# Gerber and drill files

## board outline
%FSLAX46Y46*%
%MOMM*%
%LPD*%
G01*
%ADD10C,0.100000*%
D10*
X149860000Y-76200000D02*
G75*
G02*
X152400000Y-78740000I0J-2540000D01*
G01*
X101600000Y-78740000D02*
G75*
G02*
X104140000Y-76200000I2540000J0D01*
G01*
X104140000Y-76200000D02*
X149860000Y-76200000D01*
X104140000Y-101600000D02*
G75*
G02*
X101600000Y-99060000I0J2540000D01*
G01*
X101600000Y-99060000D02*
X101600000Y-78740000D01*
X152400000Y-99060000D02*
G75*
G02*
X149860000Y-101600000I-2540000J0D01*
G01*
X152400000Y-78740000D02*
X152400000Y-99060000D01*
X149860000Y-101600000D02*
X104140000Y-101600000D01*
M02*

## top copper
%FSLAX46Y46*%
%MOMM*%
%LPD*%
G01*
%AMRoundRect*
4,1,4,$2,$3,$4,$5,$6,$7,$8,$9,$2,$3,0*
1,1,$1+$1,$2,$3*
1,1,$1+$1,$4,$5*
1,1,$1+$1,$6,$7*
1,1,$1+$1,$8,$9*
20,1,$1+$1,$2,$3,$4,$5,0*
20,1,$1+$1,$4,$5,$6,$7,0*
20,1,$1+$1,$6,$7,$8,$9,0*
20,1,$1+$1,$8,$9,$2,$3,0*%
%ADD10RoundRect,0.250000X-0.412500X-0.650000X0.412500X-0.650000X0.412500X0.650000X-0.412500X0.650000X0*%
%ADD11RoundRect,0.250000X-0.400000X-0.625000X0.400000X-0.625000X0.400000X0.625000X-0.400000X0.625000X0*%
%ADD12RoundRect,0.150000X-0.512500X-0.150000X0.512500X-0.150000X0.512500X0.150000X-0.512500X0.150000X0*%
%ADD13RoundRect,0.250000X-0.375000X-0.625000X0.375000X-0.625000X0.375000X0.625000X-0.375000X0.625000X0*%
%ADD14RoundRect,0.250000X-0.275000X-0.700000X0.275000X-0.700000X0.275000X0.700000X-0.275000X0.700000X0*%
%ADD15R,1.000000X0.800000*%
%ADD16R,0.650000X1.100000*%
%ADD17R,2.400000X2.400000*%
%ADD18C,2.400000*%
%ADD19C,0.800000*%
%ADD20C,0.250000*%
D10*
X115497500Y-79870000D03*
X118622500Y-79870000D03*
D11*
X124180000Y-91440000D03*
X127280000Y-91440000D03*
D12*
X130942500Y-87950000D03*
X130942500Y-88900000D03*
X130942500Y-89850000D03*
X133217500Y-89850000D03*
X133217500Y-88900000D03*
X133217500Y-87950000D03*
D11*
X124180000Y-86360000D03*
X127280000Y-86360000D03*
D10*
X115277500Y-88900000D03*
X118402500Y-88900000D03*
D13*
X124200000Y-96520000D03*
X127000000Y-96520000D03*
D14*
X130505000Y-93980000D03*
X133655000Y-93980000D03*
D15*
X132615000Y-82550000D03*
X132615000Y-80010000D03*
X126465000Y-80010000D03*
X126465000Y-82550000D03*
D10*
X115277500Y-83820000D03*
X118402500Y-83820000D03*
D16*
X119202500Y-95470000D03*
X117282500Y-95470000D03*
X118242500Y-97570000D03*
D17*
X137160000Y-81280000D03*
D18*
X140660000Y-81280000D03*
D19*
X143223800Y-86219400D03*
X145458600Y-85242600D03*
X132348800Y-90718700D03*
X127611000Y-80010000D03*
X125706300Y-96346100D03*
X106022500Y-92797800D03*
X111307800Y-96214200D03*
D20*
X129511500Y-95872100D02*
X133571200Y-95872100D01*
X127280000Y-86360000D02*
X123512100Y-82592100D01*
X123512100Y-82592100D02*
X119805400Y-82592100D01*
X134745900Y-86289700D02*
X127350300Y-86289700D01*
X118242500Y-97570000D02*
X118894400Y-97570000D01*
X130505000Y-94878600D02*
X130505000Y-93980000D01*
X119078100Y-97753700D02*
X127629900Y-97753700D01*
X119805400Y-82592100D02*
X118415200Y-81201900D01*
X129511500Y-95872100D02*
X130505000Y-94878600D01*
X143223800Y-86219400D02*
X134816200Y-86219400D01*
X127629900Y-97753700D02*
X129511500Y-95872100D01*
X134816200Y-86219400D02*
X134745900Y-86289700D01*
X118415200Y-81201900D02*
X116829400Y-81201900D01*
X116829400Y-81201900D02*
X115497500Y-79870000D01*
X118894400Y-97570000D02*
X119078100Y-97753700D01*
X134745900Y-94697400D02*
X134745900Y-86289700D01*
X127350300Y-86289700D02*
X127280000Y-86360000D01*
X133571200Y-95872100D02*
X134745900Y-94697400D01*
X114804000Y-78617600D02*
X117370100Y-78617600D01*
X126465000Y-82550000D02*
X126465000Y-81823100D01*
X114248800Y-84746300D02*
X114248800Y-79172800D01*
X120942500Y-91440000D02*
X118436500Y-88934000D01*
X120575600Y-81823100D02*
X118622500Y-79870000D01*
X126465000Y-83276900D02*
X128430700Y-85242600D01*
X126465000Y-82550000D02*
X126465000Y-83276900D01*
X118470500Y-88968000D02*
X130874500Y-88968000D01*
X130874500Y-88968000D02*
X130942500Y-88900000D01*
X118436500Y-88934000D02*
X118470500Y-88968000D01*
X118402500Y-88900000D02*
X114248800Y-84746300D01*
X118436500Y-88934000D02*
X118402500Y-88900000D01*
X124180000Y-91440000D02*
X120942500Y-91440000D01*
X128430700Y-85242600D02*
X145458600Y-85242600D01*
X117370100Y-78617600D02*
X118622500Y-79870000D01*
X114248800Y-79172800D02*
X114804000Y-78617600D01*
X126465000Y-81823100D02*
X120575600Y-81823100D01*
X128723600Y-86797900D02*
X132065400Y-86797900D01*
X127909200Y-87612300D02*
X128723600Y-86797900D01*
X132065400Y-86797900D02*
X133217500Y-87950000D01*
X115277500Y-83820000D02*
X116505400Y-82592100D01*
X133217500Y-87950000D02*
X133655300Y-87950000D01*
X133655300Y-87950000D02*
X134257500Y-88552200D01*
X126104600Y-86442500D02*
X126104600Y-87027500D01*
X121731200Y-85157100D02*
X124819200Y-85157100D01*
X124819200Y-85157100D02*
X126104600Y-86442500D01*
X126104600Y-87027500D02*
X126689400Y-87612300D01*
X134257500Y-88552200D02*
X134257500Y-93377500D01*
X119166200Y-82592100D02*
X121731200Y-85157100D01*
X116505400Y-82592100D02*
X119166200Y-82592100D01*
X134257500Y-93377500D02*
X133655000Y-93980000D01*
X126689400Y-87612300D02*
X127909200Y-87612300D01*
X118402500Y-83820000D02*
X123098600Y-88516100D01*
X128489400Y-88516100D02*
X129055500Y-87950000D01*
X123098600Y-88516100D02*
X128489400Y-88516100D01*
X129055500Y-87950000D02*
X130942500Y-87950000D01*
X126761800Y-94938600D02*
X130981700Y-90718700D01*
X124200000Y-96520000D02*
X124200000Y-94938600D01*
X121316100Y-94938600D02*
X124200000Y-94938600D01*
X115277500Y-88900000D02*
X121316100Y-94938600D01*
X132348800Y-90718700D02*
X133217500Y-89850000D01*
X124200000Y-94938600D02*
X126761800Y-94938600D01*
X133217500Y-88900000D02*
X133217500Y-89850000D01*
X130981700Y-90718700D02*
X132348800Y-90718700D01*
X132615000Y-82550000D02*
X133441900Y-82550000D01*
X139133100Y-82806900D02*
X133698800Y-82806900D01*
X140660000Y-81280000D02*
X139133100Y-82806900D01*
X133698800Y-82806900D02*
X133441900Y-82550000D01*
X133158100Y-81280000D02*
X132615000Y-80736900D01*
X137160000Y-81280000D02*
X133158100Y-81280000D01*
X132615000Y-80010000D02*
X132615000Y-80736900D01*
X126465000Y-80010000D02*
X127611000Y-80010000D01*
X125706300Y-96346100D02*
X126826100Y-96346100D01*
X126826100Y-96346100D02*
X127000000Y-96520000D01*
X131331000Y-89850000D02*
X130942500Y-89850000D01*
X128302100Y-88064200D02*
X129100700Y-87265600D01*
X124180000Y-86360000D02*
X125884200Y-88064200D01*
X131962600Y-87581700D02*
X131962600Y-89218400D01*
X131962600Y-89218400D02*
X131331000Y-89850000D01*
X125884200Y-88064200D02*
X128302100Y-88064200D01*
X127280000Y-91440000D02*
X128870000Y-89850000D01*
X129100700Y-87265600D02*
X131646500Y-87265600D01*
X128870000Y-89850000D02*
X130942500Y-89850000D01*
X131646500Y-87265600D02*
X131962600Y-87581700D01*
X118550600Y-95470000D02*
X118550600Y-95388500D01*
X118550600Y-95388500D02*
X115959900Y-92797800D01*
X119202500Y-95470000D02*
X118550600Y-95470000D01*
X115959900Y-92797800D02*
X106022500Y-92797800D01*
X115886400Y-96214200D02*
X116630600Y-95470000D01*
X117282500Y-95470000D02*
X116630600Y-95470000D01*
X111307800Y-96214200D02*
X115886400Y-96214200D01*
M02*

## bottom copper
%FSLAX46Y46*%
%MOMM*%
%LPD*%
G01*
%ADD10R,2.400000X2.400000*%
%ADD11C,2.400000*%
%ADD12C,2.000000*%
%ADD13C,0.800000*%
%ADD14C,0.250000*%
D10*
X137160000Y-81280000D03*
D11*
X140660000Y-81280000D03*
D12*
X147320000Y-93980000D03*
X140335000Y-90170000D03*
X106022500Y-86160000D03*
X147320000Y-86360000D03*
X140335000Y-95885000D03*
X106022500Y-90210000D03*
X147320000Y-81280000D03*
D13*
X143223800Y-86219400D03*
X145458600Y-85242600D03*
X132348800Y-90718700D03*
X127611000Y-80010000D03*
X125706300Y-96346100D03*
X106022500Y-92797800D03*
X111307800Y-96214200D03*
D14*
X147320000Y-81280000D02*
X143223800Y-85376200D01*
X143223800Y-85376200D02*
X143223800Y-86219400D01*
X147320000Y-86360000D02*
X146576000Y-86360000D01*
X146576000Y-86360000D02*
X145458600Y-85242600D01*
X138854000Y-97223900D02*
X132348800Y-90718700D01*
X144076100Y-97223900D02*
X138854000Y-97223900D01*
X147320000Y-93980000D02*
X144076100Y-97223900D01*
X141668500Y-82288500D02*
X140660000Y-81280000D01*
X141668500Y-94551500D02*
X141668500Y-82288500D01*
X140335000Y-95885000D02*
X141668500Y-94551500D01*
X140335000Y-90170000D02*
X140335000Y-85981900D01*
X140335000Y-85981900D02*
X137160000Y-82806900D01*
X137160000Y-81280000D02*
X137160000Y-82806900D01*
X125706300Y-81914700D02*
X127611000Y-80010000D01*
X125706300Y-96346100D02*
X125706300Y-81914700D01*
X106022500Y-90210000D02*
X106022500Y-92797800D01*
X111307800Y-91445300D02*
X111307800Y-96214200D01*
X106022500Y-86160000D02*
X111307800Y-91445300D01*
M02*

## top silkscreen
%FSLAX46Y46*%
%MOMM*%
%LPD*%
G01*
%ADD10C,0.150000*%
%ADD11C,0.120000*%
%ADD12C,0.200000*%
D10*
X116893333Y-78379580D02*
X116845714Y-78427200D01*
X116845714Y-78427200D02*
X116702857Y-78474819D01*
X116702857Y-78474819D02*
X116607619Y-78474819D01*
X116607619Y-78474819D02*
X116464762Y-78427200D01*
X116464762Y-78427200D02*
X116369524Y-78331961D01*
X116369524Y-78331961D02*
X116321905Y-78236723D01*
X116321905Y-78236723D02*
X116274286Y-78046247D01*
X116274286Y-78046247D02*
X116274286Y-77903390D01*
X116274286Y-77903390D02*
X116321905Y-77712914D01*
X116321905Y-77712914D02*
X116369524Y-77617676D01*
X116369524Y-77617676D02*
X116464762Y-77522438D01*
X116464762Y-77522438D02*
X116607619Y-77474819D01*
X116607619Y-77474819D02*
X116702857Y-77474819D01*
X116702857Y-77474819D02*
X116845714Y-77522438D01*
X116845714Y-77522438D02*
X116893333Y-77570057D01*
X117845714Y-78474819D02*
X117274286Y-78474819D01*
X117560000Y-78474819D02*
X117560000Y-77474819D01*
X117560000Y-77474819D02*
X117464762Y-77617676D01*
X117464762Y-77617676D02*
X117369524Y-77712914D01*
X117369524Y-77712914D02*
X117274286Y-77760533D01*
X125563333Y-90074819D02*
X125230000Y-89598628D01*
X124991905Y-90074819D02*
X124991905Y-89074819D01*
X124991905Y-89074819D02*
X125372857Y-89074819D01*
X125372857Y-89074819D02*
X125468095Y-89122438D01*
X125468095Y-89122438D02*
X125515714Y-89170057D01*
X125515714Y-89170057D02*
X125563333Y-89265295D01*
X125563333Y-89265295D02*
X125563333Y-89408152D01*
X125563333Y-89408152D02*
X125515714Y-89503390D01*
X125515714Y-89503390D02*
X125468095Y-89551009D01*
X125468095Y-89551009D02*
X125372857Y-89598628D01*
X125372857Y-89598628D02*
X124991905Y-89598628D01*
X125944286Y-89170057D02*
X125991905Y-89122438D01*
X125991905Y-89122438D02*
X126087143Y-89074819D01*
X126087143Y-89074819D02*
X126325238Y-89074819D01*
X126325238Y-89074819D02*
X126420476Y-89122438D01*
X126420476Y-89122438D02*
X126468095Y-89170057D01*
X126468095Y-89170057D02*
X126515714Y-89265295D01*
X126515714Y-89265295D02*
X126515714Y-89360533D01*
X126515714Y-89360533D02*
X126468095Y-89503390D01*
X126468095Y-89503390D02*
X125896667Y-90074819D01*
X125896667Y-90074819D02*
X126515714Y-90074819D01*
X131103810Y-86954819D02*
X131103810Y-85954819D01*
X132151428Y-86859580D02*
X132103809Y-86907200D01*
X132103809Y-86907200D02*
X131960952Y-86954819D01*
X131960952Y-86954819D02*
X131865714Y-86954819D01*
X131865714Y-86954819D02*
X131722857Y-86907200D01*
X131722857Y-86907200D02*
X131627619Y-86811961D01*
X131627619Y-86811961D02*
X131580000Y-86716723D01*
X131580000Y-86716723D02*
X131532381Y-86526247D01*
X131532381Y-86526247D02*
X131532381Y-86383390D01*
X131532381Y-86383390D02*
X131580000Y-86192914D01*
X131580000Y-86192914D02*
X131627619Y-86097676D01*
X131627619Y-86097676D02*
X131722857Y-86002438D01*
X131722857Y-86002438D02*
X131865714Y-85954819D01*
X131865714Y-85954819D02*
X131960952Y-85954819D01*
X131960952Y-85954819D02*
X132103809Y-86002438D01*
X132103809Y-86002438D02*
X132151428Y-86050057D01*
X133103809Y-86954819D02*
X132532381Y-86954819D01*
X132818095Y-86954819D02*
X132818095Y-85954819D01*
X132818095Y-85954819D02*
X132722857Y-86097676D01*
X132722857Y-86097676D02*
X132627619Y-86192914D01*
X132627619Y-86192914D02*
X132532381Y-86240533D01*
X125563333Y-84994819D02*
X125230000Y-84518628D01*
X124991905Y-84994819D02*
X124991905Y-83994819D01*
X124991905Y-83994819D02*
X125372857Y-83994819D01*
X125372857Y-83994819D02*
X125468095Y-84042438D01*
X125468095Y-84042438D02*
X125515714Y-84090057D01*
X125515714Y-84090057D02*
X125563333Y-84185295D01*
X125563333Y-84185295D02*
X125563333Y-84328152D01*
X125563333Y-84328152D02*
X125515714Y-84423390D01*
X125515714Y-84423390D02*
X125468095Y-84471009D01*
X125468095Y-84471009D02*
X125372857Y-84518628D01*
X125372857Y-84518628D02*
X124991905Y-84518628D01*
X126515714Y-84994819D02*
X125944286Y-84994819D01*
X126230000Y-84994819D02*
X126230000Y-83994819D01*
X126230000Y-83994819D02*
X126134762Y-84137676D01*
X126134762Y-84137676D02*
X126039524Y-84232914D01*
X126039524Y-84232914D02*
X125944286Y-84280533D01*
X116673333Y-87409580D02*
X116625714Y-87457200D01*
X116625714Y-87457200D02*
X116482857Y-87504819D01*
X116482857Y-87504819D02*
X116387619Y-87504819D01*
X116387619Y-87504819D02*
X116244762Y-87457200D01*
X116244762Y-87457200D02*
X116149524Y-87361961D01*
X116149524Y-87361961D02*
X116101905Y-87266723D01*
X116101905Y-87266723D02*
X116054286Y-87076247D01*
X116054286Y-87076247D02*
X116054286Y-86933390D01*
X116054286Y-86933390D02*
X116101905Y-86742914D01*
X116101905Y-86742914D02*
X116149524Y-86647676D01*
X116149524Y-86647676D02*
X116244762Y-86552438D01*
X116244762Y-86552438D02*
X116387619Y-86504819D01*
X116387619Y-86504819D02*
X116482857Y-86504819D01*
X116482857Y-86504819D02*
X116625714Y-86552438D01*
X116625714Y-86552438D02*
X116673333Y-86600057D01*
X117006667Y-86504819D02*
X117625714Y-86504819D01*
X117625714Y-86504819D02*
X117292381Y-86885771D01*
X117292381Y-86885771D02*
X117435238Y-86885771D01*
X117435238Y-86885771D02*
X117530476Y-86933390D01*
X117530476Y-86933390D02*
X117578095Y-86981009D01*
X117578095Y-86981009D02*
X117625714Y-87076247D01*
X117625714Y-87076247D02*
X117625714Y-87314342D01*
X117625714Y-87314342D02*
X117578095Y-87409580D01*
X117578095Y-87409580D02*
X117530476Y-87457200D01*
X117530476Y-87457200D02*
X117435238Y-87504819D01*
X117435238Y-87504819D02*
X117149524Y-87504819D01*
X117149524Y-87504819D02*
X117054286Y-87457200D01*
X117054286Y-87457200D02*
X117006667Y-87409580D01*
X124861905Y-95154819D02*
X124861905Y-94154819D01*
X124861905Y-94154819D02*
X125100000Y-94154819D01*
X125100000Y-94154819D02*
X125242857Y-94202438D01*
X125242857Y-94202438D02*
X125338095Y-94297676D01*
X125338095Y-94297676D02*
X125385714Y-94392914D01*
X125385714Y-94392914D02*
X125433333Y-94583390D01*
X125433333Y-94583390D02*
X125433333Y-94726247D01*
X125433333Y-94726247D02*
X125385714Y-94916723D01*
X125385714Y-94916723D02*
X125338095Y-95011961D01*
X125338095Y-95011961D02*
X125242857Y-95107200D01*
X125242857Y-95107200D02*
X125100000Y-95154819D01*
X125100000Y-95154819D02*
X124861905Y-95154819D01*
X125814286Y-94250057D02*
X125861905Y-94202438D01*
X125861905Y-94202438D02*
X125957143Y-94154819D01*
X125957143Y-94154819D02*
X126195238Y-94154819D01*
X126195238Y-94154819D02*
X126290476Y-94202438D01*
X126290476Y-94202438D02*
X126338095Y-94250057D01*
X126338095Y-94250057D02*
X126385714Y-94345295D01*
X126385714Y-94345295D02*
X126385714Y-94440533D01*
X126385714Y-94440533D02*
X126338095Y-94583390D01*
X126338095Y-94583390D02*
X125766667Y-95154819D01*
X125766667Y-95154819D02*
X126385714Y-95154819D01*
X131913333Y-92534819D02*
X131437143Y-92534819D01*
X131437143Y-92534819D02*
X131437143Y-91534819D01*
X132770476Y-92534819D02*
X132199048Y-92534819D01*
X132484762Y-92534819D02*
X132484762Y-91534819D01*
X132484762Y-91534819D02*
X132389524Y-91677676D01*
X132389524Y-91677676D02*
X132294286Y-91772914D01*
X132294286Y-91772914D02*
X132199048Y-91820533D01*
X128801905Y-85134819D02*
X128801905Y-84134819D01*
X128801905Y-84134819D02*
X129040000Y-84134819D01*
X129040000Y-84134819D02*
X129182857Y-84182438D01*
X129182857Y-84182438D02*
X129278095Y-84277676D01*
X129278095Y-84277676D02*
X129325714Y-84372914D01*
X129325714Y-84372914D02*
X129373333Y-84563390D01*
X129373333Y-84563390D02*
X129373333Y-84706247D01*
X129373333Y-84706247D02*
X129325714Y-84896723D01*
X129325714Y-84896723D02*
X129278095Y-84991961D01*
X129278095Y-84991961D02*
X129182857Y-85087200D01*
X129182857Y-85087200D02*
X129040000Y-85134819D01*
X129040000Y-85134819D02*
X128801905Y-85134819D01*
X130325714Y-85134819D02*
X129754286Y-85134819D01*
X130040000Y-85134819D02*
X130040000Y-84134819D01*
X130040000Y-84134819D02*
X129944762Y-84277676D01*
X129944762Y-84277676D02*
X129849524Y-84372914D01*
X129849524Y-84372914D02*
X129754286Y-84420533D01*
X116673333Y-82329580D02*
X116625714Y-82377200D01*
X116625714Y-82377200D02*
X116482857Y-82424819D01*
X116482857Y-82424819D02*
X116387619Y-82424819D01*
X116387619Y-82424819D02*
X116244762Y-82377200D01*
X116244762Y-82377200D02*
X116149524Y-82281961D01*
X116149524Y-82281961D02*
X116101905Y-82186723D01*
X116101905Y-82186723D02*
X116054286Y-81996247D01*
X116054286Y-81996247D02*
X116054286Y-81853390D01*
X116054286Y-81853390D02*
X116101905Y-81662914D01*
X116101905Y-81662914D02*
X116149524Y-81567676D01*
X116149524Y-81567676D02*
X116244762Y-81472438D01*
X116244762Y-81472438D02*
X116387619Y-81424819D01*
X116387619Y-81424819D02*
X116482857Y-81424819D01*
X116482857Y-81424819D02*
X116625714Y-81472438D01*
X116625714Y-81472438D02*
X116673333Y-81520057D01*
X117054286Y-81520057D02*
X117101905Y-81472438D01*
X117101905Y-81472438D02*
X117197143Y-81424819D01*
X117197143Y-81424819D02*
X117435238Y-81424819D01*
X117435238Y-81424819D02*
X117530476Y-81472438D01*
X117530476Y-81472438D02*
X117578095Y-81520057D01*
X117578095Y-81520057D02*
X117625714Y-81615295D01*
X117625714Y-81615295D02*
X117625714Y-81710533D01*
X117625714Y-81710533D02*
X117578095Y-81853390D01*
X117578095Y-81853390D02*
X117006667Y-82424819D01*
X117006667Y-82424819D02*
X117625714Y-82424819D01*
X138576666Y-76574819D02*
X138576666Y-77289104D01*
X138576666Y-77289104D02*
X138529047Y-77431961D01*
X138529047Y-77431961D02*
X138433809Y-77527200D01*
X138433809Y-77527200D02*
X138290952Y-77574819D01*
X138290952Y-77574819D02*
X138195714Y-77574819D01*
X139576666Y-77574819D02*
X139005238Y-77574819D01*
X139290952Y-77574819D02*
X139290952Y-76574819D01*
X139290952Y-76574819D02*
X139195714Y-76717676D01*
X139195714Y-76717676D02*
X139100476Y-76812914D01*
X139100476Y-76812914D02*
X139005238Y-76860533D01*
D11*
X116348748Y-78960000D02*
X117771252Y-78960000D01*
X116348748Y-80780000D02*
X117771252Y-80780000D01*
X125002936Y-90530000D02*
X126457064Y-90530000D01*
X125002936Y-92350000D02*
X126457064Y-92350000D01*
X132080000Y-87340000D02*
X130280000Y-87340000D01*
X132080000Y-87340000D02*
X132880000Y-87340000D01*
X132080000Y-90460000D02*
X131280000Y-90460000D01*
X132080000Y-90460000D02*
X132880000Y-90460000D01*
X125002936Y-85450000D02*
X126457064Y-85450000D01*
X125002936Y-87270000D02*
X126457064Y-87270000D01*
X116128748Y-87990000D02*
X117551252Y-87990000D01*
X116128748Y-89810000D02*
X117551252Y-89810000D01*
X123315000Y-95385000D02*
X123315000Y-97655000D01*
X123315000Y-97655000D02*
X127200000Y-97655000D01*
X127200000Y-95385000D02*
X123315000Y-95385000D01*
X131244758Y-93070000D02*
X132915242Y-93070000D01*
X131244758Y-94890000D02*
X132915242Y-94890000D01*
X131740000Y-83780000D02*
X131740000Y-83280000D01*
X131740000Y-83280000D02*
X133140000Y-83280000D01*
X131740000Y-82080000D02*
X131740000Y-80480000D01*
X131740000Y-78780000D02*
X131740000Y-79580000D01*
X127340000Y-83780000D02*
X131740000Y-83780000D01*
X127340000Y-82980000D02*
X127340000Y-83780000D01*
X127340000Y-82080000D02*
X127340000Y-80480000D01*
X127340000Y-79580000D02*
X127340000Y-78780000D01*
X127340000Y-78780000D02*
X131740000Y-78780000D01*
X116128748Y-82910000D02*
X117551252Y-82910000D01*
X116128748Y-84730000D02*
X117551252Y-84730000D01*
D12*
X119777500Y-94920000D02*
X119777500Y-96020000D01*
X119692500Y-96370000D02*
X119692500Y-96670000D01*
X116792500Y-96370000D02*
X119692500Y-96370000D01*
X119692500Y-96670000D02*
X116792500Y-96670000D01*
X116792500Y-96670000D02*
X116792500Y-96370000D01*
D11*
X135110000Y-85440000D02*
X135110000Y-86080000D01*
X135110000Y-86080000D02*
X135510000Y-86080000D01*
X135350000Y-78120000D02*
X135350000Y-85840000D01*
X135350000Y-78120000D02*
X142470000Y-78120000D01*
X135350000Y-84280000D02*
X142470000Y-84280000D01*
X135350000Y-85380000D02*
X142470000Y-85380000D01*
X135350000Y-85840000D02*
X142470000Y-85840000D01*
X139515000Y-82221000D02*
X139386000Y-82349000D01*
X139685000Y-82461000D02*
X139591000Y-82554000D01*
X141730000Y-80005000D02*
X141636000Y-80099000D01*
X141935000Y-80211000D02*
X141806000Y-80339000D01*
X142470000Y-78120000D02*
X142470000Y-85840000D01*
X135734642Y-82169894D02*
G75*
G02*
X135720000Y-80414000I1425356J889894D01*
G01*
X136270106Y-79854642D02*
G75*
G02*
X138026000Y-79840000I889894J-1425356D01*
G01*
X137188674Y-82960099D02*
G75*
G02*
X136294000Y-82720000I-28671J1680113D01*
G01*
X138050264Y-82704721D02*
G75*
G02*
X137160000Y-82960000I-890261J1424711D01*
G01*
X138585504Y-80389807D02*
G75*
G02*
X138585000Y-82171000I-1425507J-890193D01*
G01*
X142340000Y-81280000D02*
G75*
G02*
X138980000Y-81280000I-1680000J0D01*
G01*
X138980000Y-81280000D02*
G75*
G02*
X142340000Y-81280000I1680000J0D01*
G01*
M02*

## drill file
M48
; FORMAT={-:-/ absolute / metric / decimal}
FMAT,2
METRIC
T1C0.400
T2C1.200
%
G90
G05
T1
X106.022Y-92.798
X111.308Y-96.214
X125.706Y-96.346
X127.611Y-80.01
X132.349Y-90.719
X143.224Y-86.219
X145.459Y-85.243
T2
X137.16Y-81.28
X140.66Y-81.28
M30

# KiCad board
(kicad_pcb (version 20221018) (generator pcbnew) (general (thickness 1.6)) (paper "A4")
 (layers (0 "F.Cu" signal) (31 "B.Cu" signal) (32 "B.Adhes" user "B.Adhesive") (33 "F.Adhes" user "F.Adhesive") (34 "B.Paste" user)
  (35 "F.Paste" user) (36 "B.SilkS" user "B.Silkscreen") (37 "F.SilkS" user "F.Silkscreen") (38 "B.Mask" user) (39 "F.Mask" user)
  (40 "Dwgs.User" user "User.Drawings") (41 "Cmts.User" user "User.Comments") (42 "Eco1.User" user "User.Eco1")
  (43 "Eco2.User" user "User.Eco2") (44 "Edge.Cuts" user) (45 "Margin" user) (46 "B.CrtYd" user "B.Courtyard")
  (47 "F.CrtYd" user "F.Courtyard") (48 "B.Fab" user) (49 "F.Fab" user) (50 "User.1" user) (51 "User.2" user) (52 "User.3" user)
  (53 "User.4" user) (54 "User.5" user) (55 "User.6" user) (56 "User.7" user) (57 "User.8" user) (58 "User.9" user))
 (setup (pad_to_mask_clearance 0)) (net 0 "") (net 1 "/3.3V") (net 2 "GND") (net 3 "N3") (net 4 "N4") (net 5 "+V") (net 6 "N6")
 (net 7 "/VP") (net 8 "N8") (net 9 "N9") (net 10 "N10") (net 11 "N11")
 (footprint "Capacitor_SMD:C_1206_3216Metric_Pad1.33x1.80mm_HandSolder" (layer "F.Cu") (at 117.06 79.87)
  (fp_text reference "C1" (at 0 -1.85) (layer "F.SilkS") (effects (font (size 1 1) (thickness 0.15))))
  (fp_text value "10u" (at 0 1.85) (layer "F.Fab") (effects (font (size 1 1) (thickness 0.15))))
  (fp_line (start -0.711252 -0.91) (end 0.711252 -0.91) (stroke (width 0.12) (type solid)) (layer "F.SilkS"))
  (fp_line (start -0.711252 0.91) (end 0.711252 0.91) (stroke (width 0.12) (type solid)) (layer "F.SilkS"))
  (pad "1" smd roundrect (at -1.5625 0) (size 1.325 1.8) (layers "F.Cu" "F.Paste" "F.Mask") (roundrect_rratio 0.1886792453) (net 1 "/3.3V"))
  (pad "2" smd roundrect (at 1.5625 0) (size 1.325 1.8) (layers "F.Cu" "F.Paste" "F.Mask") (roundrect_rratio 0.1886792453) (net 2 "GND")))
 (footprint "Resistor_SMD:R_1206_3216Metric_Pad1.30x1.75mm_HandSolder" (layer "F.Cu") (at 125.73 91.44)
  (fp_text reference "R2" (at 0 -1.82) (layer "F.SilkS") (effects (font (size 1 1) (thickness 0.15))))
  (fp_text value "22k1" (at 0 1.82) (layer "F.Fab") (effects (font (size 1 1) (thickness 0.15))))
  (fp_line (start -0.727064 -0.91) (end 0.727064 -0.91) (stroke (width 0.12) (type solid)) (layer "F.SilkS"))
  (fp_line (start -0.727064 0.91) (end 0.727064 0.91) (stroke (width 0.12) (type solid)) (layer "F.SilkS"))
  (pad "1" smd roundrect (at -1.55 0) (size 1.3 1.75) (layers "F.Cu" "F.Paste" "F.Mask") (roundrect_rratio 0.1923076923) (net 2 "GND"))
  (pad "2" smd roundrect (at 1.55 0) (size 1.3 1.75) (layers "F.Cu" "F.Paste" "F.Mask") (roundrect_rratio 0.1923076923) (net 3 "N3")))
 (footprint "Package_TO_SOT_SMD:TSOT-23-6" (layer "F.Cu") (at 132.08 88.9)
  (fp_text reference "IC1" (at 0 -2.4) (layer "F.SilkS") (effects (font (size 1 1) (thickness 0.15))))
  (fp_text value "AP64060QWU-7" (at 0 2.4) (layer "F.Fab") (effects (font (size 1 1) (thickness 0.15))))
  (fp_line (start 0 -1.56) (end -1.8 -1.56) (stroke (width 0.12) (type solid)) (layer "F.SilkS"))
  (fp_line (start 0 -1.56) (end 0.8 -1.56) (stroke (width 0.12) (type solid)) (layer "F.SilkS"))
  (fp_line (start 0 1.56) (end -0.8 1.56) (stroke (width 0.12) (type solid)) (layer "F.SilkS"))
  (fp_line (start 0 1.56) (end 0.8 1.56) (stroke (width 0.12) (type solid)) (layer "F.SilkS"))
  (pad "1" smd roundrect (at -1.1375 -0.95) (size 1.325 0.6) (layers "F.Cu" "F.Paste" "F.Mask") (roundrect_rratio 0.25) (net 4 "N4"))
  (pad "2" smd roundrect (at -1.1375 0) (size 1.325 0.6) (layers "F.Cu" "F.Paste" "F.Mask") (roundrect_rratio 0.25) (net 2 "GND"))
  (pad "3" smd roundrect (at -1.1375 0.95) (size 1.325 0.6) (layers "F.Cu" "F.Paste" "F.Mask") (roundrect_rratio 0.25) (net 3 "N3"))
  (pad "4" smd roundrect (at 1.1375 0.95) (size 1.325 0.6) (layers "F.Cu" "F.Paste" "F.Mask") (roundrect_rratio 0.25) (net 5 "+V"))
  (pad "5" smd roundrect (at 1.1375 0) (size 1.325 0.6) (layers "F.Cu" "F.Paste" "F.Mask") (roundrect_rratio 0.25) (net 5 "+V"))
  (pad "6" smd roundrect (at 1.1375 -0.95) (size 1.325 0.6) (layers "F.Cu" "F.Paste" "F.Mask") (roundrect_rratio 0.25) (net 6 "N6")))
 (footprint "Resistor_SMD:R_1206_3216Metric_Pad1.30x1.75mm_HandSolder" (layer "F.Cu") (at 125.73 86.36)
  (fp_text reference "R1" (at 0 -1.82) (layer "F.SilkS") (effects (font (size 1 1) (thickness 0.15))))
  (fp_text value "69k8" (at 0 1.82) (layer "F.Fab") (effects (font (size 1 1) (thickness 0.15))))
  (fp_line (start -0.727064 -0.91) (end 0.727064 -0.91) (stroke (width 0.12) (type solid)) (layer "F.SilkS"))
  (fp_line (start -0.727064 0.91) (end 0.727064 0.91) (stroke (width 0.12) (type solid)) (layer "F.SilkS"))
  (pad "1" smd roundrect (at -1.55 0) (size 1.3 1.75) (layers "F.Cu" "F.Paste" "F.Mask") (roundrect_rratio 0.1923076923) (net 3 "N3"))
  (pad "2" smd roundrect (at 1.55 0) (size 1.3 1.75) (layers "F.Cu" "F.Paste" "F.Mask") (roundrect_rratio 0.1923076923) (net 1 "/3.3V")))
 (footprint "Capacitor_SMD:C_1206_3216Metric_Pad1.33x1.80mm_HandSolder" (layer "F.Cu") (at 116.84 88.9)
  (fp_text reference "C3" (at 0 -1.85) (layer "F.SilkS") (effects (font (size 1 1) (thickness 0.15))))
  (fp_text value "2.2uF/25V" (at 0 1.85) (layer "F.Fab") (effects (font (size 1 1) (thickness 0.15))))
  (fp_line (start -0.711252 -0.91) (end 0.711252 -0.91) (stroke (width 0.12) (type solid)) (layer "F.SilkS"))
  (fp_line (start -0.711252 0.91) (end 0.711252 0.91) (stroke (width 0.12) (type solid)) (layer "F.SilkS"))
  (pad "1" smd roundrect (at -1.5625 0) (size 1.325 1.8) (layers "F.Cu" "F.Paste" "F.Mask") (roundrect_rratio 0.1886792453) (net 5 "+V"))
  (pad "2" smd roundrect (at 1.5625 0) (size 1.325 1.8) (layers "F.Cu" "F.Paste" "F.Mask") (roundrect_rratio 0.1886792453) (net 2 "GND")))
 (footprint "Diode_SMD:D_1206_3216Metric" (layer "F.Cu") (at 125.6 96.52)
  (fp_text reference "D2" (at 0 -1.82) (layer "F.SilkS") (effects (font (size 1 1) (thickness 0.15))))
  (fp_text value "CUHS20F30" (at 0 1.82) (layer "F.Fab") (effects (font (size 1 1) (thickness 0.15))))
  (fp_line (start -2.285 -1.135) (end -2.285 1.135) (stroke (width 0.12) (type solid)) (layer "F.SilkS"))
  (fp_line (start -2.285 1.135) (end 1.6 1.135) (stroke (width 0.12) (type solid)) (layer "F.SilkS"))
  (fp_line (start 1.6 -1.135) (end -2.285 -1.135) (stroke (width 0.12) (type solid)) (layer "F.SilkS"))
  (pad "1" smd roundrect (at -1.4 0) (size 1.25 1.75) (layers "F.Cu" "F.Paste" "F.Mask") (roundrect_rratio 0.2) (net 5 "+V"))
  (pad "2" smd roundrect (at 1.4 0) (size 1.25 1.75) (layers "F.Cu" "F.Paste" "F.Mask") (roundrect_rratio 0.2) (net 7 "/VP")))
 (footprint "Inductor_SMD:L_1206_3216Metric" (layer "F.Cu") (at 132.08 93.98)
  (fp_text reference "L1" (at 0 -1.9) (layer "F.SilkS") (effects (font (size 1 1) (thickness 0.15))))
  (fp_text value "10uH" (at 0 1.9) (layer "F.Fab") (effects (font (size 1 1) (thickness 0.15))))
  (fp_line (start -0.835242 -0.91) (end 0.835242 -0.91) (stroke (width 0.12) (type solid)) (layer "F.SilkS"))
  (fp_line (start -0.835242 0.91) (end 0.835242 0.91) (stroke (width 0.12) (type solid)) (layer "F.SilkS"))
  (pad "1" smd roundrect (at -1.575 0) (size 1.05 1.9) (layers "F.Cu" "F.Paste" "F.Mask") (roundrect_rratio 0.2380952381) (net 1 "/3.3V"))
  (pad "2" smd roundrect (at 1.575 0) (size 1.05 1.9) (layers "F.Cu" "F.Paste" "F.Mask") (roundrect_rratio 0.2380952381) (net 6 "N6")))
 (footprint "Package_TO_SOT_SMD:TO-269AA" (layer "F.Cu") (at 129.54 81.28 180)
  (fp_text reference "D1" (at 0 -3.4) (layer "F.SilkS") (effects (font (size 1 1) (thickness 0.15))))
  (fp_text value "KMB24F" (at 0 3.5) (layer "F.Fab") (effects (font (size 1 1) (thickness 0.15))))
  (fp_line (start -2.2 -2.5) (end -2.2 -2) (stroke (width 0.12) (type solid)) (layer "F.SilkS"))
  (fp_line (start -2.2 -2) (end -3.6 -2) (stroke (width 0.12) (type solid)) (layer "F.SilkS"))
  (fp_line (start -2.2 -0.8) (end -2.2 0.8) (stroke (width 0.12) (type solid)) (layer "F.SilkS"))
  (fp_line (start -2.2 2.5) (end -2.2 1.7) (stroke (width 0.12) (type solid)) (layer "F.SilkS"))
  (fp_line (start 2.2 -2.5) (end -2.2 -2.5) (stroke (width 0.12) (type solid)) (layer "F.SilkS"))
  (fp_line (start 2.2 -1.7) (end 2.2 -2.5) (stroke (width 0.12) (type solid)) (layer "F.SilkS"))
  (fp_line (start 2.2 -0.8) (end 2.2 0.8) (stroke (width 0.12) (type solid)) (layer "F.SilkS"))
  (fp_line (start 2.2 1.7) (end 2.2 2.5) (stroke (width 0.12) (type solid)) (layer "F.SilkS"))
  (fp_line (start 2.2 2.5) (end -2.2 2.5) (stroke (width 0.12) (type solid)) (layer "F.SilkS"))
  (pad "1" smd rect (at -3.075 -1.27 180) (size 1 0.8) (layers "F.Cu" "F.Paste" "F.Mask") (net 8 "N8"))
  (pad "2" smd rect (at -3.075 1.27 180) (size 1 0.8) (layers "F.Cu" "F.Paste" "F.Mask") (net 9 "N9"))
  (pad "3" smd rect (at 3.075 1.27 180) (size 1 0.8) (layers "F.Cu" "F.Paste" "F.Mask") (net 7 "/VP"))
  (pad "4" smd rect (at 3.075 -1.27 180) (size 1 0.8) (layers "F.Cu" "F.Paste" "F.Mask") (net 2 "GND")))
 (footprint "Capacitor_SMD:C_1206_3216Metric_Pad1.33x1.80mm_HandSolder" (layer "F.Cu") (at 116.84 83.82)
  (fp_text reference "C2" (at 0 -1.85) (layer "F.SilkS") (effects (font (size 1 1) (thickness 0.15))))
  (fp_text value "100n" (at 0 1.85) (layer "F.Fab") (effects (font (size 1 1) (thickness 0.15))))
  (fp_line (start -0.711252 -0.91) (end 0.711252 -0.91) (stroke (width 0.12) (type solid)) (layer "F.SilkS"))
  (fp_line (start -0.711252 0.91) (end 0.711252 0.91) (stroke (width 0.12) (type solid)) (layer "F.SilkS"))
  (pad "1" smd roundrect (at -1.5625 0) (size 1.325 1.8) (layers "F.Cu" "F.Paste" "F.Mask") (roundrect_rratio 0.1886792453) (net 6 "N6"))
  (pad "2" smd roundrect (at 1.5625 0) (size 1.325 1.8) (layers "F.Cu" "F.Paste" "F.Mask") (roundrect_rratio 0.1886792453) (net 4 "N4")))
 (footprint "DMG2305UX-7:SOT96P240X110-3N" (layer "F.Cu") (at 118.2425 96.52 -90)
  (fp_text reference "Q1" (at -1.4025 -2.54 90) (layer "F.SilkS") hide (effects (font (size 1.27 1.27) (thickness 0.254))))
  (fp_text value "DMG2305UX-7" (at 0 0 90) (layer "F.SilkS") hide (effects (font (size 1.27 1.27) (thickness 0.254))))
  (fp_line (start -1.6 -1.535) (end -0.5 -1.535) (stroke (width 0.2) (type solid)) (layer "F.SilkS"))
  (fp_line (start -0.15 -1.45) (end 0.15 -1.45) (stroke (width 0.2) (type solid)) (layer "F.SilkS"))
  (fp_line (start -0.15 1.45) (end -0.15 -1.45) (stroke (width 0.2) (type solid)) (layer "F.SilkS"))
  (fp_line (start 0.15 -1.45) (end 0.15 1.45) (stroke (width 0.2) (type solid)) (layer "F.SilkS"))
  (fp_line (start 0.15 1.45) (end -0.15 1.45) (stroke (width 0.2) (type solid)) (layer "F.SilkS"))
  (pad "1" smd rect (at -1.05 -0.96) (size 0.65 1.1) (layers "F.Cu" "F.Paste" "F.Mask") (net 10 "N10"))
  (pad "2" smd rect (at -1.05 0.96) (size 0.65 1.1) (layers "F.Cu" "F.Paste" "F.Mask") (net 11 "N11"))
  (pad "3" smd rect (at 1.05 0) (size 0.65 1.1) (layers "F.Cu" "F.Paste" "F.Mask") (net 1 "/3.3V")))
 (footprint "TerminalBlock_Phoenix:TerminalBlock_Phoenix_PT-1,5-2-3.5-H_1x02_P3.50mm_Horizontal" (layer "F.Cu") (at 137.16 81.28)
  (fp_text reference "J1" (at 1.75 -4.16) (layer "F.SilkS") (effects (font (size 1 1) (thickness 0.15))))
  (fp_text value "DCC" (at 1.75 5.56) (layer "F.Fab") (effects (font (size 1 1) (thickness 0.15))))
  (fp_line (start -2.05 4.16) (end -2.05 4.8) (stroke (width 0.12) (type solid)) (layer "F.SilkS"))
  (fp_line (start -2.05 4.8) (end -1.65 4.8) (stroke (width 0.12) (type solid)) (layer "F.SilkS"))
  (fp_line (start -1.81 -3.16) (end -1.81 4.56) (stroke (width 0.12) (type solid)) (layer "F.SilkS"))
  (fp_line (start -1.81 -3.16) (end 5.31 -3.16) (stroke (width 0.12) (type solid)) (layer "F.SilkS"))
  (fp_line (start -1.81 3) (end 5.31 3) (stroke (width 0.12) (type solid)) (layer "F.SilkS"))
  (fp_line (start -1.81 4.1) (end 5.31 4.1) (stroke (width 0.12) (type solid)) (layer "F.SilkS"))
  (fp_line (start -1.81 4.56) (end 5.31 4.56) (stroke (width 0.12) (type solid)) (layer "F.SilkS"))
  (fp_line (start 2.355 0.941) (end 2.226 1.069) (stroke (width 0.12) (type solid)) (layer "F.SilkS"))
  (fp_line (start 2.525 1.181) (end 2.431 1.274) (stroke (width 0.12) (type solid)) (layer "F.SilkS"))
  (fp_line (start 4.57 -1.275) (end 4.476 -1.181) (stroke (width 0.12) (type solid)) (layer "F.SilkS"))
  (fp_line (start 4.775 -1.069) (end 4.646 -0.941) (stroke (width 0.12) (type solid)) (layer "F.SilkS"))
  (fp_line (start 5.31 -3.16) (end 5.31 4.56) (stroke (width 0.12) (type solid)) (layer "F.SilkS"))
  (fp_arc (start -1.425358 0.889894) (mid -1.680286 0.014012) (end -1.44 -0.866) (stroke (width 0.12) (type solid)) (layer "F.SilkS"))
  (fp_arc (start -0.889894 -1.425358) (mid -0.014012 -1.680286) (end 0.866 -1.44) (stroke (width 0.12) (type solid)) (layer "F.SilkS"))
  (fp_arc (start 0.028674 1.680099) (mid -0.435535 1.622918) (end -0.866 1.44) (stroke (width 0.12) (type solid)) (layer "F.SilkS"))
  (fp_arc (start 0.890264 1.424721) (mid 0.463071 1.61492) (end 0 1.68) (stroke (width 0.12) (type solid)) (layer "F.SilkS"))
  (fp_arc (start 1.425504 -0.890193) (mid 1.680626 0.000476) (end 1.425 0.891) (stroke (width 0.12) (type solid)) (layer "F.SilkS"))
  (fp_circle (center 3.5 0) (end 5.18 0) (stroke (width 0.12) (type solid)) (fill none) (layer "F.SilkS"))
  (pad "1" thru_hole rect (at 0 0) (size 2.4 2.4) (drill 1.2) (layers "*.Cu" "*.Mask") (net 9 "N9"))
  (pad "2" thru_hole circle (at 3.5 0) (size 2.4 2.4) (drill 1.2) (layers "*.Cu" "*.Mask") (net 8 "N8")))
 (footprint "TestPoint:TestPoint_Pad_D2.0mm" (layer "B.Cu") (at 147.32 93.98 180)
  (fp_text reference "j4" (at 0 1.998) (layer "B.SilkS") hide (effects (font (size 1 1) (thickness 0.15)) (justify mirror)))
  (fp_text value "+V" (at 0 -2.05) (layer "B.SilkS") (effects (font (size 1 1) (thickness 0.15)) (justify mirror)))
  (pad "1" smd circle (at 0 0 180) (size 2 2) (layers "B.Cu" "B.Mask") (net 5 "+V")))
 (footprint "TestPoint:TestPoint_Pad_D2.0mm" (layer "B.Cu") (at 140.335 90.17 180)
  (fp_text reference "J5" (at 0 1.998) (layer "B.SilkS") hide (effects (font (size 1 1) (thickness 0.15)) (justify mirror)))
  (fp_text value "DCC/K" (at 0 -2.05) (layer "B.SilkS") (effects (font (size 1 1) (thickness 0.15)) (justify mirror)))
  (pad "1" smd circle (at 0 0 180) (size 2 2) (layers "B.Cu" "B.Mask") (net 9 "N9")))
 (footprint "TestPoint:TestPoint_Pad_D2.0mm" (layer "B.Cu") (at 106.0225 86.16 180)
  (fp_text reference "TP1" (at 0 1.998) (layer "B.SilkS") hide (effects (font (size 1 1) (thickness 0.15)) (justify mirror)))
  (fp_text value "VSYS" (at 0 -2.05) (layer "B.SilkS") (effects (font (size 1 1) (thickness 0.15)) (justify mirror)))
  (pad "1" smd circle (at 0 0 180) (size 2 2) (layers "B.Cu" "B.Mask") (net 11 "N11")))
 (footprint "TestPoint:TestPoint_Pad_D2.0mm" (layer "B.Cu") (at 147.32 86.36 180)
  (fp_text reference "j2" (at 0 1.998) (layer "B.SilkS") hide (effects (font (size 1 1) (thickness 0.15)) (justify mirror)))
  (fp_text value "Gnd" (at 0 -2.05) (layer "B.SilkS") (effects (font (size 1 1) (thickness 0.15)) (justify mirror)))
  (pad "1" smd circle (at 0 0 180) (size 2 2) (layers "B.Cu" "B.Mask") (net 2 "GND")))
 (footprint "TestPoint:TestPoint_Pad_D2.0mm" (layer "B.Cu") (at 140.335 95.885 180)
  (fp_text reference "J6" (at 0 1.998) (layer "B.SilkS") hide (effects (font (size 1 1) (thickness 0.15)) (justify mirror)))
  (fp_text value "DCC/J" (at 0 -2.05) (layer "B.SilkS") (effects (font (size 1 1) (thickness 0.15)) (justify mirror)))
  (pad "1" smd circle (at 0 0 180) (size 2 2) (layers "B.Cu" "B.Mask") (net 8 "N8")))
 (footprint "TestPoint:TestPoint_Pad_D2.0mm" (layer "B.Cu") (at 106.0225 90.21 180)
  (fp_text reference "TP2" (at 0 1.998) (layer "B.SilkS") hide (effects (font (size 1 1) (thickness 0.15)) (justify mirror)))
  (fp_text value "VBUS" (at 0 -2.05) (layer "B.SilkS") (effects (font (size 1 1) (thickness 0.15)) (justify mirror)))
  (pad "1" smd circle (at 0 0 180) (size 2 2) (layers "B.Cu" "B.Mask") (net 10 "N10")))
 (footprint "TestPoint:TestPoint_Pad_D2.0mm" (layer "B.Cu") (at 147.32 81.28 180)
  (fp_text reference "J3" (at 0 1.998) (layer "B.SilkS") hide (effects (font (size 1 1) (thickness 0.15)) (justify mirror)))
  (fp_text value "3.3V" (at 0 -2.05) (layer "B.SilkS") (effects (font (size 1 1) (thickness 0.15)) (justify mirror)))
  (pad "1" smd circle (at 0 0 180) (size 2 2) (layers "B.Cu" "B.Mask") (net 1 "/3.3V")))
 (gr_arc (start 149.86 76.2) (mid 151.656051 76.943949) (end 152.4 78.74) (stroke (width 0.1) (type default)) (layer "Edge.Cuts"))
 (gr_arc (start 101.6 78.74) (mid 102.343949 76.943949) (end 104.14 76.2) (stroke (width 0.1) (type default)) (layer "Edge.Cuts"))
 (gr_line (start 104.14 76.2) (end 149.86 76.2) (stroke (width 0.1) (type default)) (layer "Edge.Cuts"))
 (gr_arc (start 104.14 101.6) (mid 102.343949 100.856051) (end 101.6 99.06) (stroke (width 0.1) (type default)) (layer "Edge.Cuts"))
 (gr_line (start 101.6 99.06) (end 101.6 78.74) (stroke (width 0.1) (type default)) (layer "Edge.Cuts"))
 (gr_arc (start 152.4 99.06) (mid 151.656051 100.856051) (end 149.86 101.6) (stroke (width 0.1) (type default)) (layer "Edge.Cuts"))
 (gr_line (start 152.4 78.74) (end 152.4 99.06) (stroke (width 0.1) (type default)) (layer "Edge.Cuts"))
 (gr_line (start 149.86 101.6) (end 104.14 101.6) (stroke (width 0.1) (type default)) (layer "Edge.Cuts"))
 (segment (start 129.5115 95.8721) (end 133.5712 95.8721) (width 0.25) (layer "F.Cu") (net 1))
 (segment (start 127.28 86.36) (end 123.5121 82.5921) (width 0.25) (layer "F.Cu") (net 1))
 (segment (start 123.5121 82.5921) (end 119.8054 82.5921) (width 0.25) (layer "F.Cu") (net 1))
 (segment (start 134.7459 86.2897) (end 127.3503 86.2897) (width 0.25) (layer "F.Cu") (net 1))
 (segment (start 118.2425 97.57) (end 118.8944 97.57) (width 0.25) (layer "F.Cu") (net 1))
 (segment (start 130.505 94.8786) (end 130.505 93.98) (width 0.25) (layer "F.Cu") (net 1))
 (segment (start 119.0781 97.7537) (end 127.6299 97.7537) (width 0.25) (layer "F.Cu") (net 1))
 (segment (start 119.8054 82.5921) (end 118.4152 81.2019) (width 0.25) (layer "F.Cu") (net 1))
 (segment (start 129.5115 95.8721) (end 130.505 94.8786) (width 0.25) (layer "F.Cu") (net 1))
 (segment (start 143.2238 86.2194) (end 134.8162 86.2194) (width 0.25) (layer "F.Cu") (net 1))
 (segment (start 127.6299 97.7537) (end 129.5115 95.8721) (width 0.25) (layer "F.Cu") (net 1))
 (segment (start 134.8162 86.2194) (end 134.7459 86.2897) (width 0.25) (layer "F.Cu") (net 1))
 (segment (start 118.4152 81.2019) (end 116.8294 81.2019) (width 0.25) (layer "F.Cu") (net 1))
 (segment (start 116.8294 81.2019) (end 115.4975 79.87) (width 0.25) (layer "F.Cu") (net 1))
 (segment (start 118.8944 97.57) (end 119.0781 97.7537) (width 0.25) (layer "F.Cu") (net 1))
 (segment (start 134.7459 94.6974) (end 134.7459 86.2897) (width 0.25) (layer "F.Cu") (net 1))
 (segment (start 127.3503 86.2897) (end 127.28 86.36) (width 0.25) (layer "F.Cu") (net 1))
 (segment (start 133.5712 95.8721) (end 134.7459 94.6974) (width 0.25) (layer "F.Cu") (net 1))
 (via (at 143.2238 86.2194) (size 0.8) (drill 0.4) (layers "F.Cu" "B.Cu") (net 1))
 (segment (start 147.32 81.28) (end 143.2238 85.3762) (width 0.25) (layer "B.Cu") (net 1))
 (segment (start 143.2238 85.3762) (end 143.2238 86.2194) (width 0.25) (layer "B.Cu") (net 1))
 (segment (start 114.804 78.6176) (end 117.3701 78.6176) (width 0.25) (layer "F.Cu") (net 2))
 (segment (start 126.465 82.55) (end 126.465 81.8231) (width 0.25) (layer "F.Cu") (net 2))
 (segment (start 114.2488 84.7463) (end 114.2488 79.1728) (width 0.25) (layer "F.Cu") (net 2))
 (segment (start 120.9425 91.44) (end 118.4365 88.934) (width 0.25) (layer "F.Cu") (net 2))
 (segment (start 120.5756 81.8231) (end 118.6225 79.87) (width 0.25) (layer "F.Cu") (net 2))
 (segment (start 126.465 83.2769) (end 128.4307 85.2426) (width 0.25) (layer "F.Cu") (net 2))
 (segment (start 126.465 82.55) (end 126.465 83.2769) (width 0.25) (layer "F.Cu") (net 2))
 (segment (start 118.4705 88.968) (end 130.8745 88.968) (width 0.25) (layer "F.Cu") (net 2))
 (segment (start 130.8745 88.968) (end 130.9425 88.9) (width 0.25) (layer "F.Cu") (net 2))
 (segment (start 118.4365 88.934) (end 118.4705 88.968) (width 0.25) (layer "F.Cu") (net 2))
 (segment (start 118.4025 88.9) (end 114.2488 84.7463) (width 0.25) (layer "F.Cu") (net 2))
 (segment (start 118.4365 88.934) (end 118.4025 88.9) (width 0.25) (layer "F.Cu") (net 2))
 (segment (start 124.18 91.44) (end 120.9425 91.44) (width 0.25) (layer "F.Cu") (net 2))
 (segment (start 128.4307 85.2426) (end 145.4586 85.2426) (width 0.25) (layer "F.Cu") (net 2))
 (segment (start 117.3701 78.6176) (end 118.6225 79.87) (width 0.25) (layer "F.Cu") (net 2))
 (segment (start 114.2488 79.1728) (end 114.804 78.6176) (width 0.25) (layer "F.Cu") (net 2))
 (segment (start 126.465 81.8231) (end 120.5756 81.8231) (width 0.25) (layer "F.Cu") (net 2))
 (via (at 145.4586 85.2426) (size 0.8) (drill 0.4) (layers "F.Cu" "B.Cu") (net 2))
 (segment (start 147.32 86.36) (end 146.576 86.36) (width 0.25) (layer "B.Cu") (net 2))
 (segment (start 146.576 86.36) (end 145.4586 85.2426) (width 0.25) (layer "B.Cu") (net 2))
 (segment (start 128.7236 86.7979) (end 132.0654 86.7979) (width 0.25) (layer "F.Cu") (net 6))
 (segment (start 127.9092 87.6123) (end 128.7236 86.7979) (width 0.25) (layer "F.Cu") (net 6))
 (segment (start 132.0654 86.7979) (end 133.2175 87.95) (width 0.25) (layer "F.Cu") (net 6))
 (segment (start 115.2775 83.82) (end 116.5054 82.5921) (width 0.25) (layer "F.Cu") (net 6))
 (segment (start 133.2175 87.95) (end 133.6553 87.95) (width 0.25) (layer "F.Cu") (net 6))
 (segment (start 133.6553 87.95) (end 134.2575 88.5522) (width 0.25) (layer "F.Cu") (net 6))
 (segment (start 126.1046 86.4425) (end 126.1046 87.0275) (width 0.25) (layer "F.Cu") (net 6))
 (segment (start 121.7312 85.1571) (end 124.8192 85.1571) (width 0.25) (layer "F.Cu") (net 6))
 (segment (start 124.8192 85.1571) (end 126.1046 86.4425) (width 0.25) (layer "F.Cu") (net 6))
 (segment (start 126.1046 87.0275) (end 126.6894 87.6123) (width 0.25) (layer "F.Cu") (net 6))
 (segment (start 134.2575 88.5522) (end 134.2575 93.3775) (width 0.25) (layer "F.Cu") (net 6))
 (segment (start 119.1662 82.5921) (end 121.7312 85.1571) (width 0.25) (layer "F.Cu") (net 6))
 (segment (start 116.5054 82.5921) (end 119.1662 82.5921) (width 0.25) (layer "F.Cu") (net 6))
 (segment (start 134.2575 93.3775) (end 133.655 93.98) (width 0.25) (layer "F.Cu") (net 6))
 (segment (start 126.6894 87.6123) (end 127.9092 87.6123) (width 0.25) (layer "F.Cu") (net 6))
 (segment (start 118.4025 83.82) (end 123.0986 88.5161) (width 0.25) (layer "F.Cu") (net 4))
 (segment (start 128.4894 88.5161) (end 129.0555 87.95) (width 0.25) (layer "F.Cu") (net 4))
 (segment (start 123.0986 88.5161) (end 128.4894 88.5161) (width 0.25) (layer "F.Cu") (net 4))
 (segment (start 129.0555 87.95) (end 130.9425 87.95) (width 0.25) (layer "F.Cu") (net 4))
 (segment (start 126.7618 94.9386) (end 130.9817 90.7187) (width 0.25) (layer "F.Cu") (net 5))
 (segment (start 124.2 96.52) (end 124.2 94.9386) (width 0.25) (layer "F.Cu") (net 5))
 (segment (start 121.3161 94.9386) (end 124.2 94.9386) (width 0.25) (layer "F.Cu") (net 5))
 (segment (start 115.2775 88.9) (end 121.3161 94.9386) (width 0.25) (layer "F.Cu") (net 5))
 (segment (start 132.3488 90.7187) (end 133.2175 89.85) (width 0.25) (layer "F.Cu") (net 5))
 (segment (start 124.2 94.9386) (end 126.7618 94.9386) (width 0.25) (layer "F.Cu") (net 5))
 (segment (start 133.2175 88.9) (end 133.2175 89.85) (width 0.25) (layer "F.Cu") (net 5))
 (segment (start 130.9817 90.7187) (end 132.3488 90.7187) (width 0.25) (layer "F.Cu") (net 5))
 (via (at 132.3488 90.7187) (size 0.8) (drill 0.4) (layers "F.Cu" "B.Cu") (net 5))
 (segment (start 138.854 97.2239) (end 132.3488 90.7187) (width 0.25) (layer "B.Cu") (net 5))
 (segment (start 144.0761 97.2239) (end 138.854 97.2239) (width 0.25) (layer "B.Cu") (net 5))
 (segment (start 147.32 93.98) (end 144.0761 97.2239) (width 0.25) (layer "B.Cu") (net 5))
 (segment (start 132.615 82.55) (end 133.4419 82.55) (width 0.25) (layer "F.Cu") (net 8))
 (segment (start 139.1331 82.8069) (end 133.6988 82.8069) (width 0.25) (layer "F.Cu") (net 8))
 (segment (start 140.66 81.28) (end 139.1331 82.8069) (width 0.25) (layer "F.Cu") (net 8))
 (segment (start 133.6988 82.8069) (end 133.4419 82.55) (width 0.25) (layer "F.Cu") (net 8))
 (segment (start 141.6685 82.2885) (end 140.66 81.28) (width 0.25) (layer "B.Cu") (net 8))
 (segment (start 141.6685 94.5515) (end 141.6685 82.2885) (width 0.25) (layer "B.Cu") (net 8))
 (segment (start 140.335 95.885) (end 141.6685 94.5515) (width 0.25) (layer "B.Cu") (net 8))
 (segment (start 133.1581 81.28) (end 132.615 80.7369) (width 0.25) (layer "F.Cu") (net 9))
 (segment (start 137.16 81.28) (end 133.1581 81.28) (width 0.25) (layer "F.Cu") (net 9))
 (segment (start 132.615 80.01) (end 132.615 80.7369) (width 0.25) (layer "F.Cu") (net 9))
 (segment (start 140.335 90.17) (end 140.335 85.9819) (width 0.25) (layer "B.Cu") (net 9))
 (segment (start 140.335 85.9819) (end 137.16 82.8069) (width 0.25) (layer "B.Cu") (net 9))
 (segment (start 137.16 81.28) (end 137.16 82.8069) (width 0.25) (layer "B.Cu") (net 9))
 (segment (start 126.465 80.01) (end 127.611 80.01) (width 0.25) (layer "F.Cu") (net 7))
 (segment (start 125.7063 96.3461) (end 126.8261 96.3461) (width 0.25) (layer "F.Cu") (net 7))
 (segment (start 126.8261 96.3461) (end 127 96.52) (width 0.25) (layer "F.Cu") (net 7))
 (via (at 127.611 80.01) (size 0.8) (drill 0.4) (layers "F.Cu" "B.Cu") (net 7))
 (via (at 125.7063 96.3461) (size 0.8) (drill 0.4) (layers "F.Cu" "B.Cu") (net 7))
 (segment (start 125.7063 81.9147) (end 127.611 80.01) (width 0.25) (layer "B.Cu") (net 7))
 (segment (start 125.7063 96.3461) (end 125.7063 81.9147) (width 0.25) (layer "B.Cu") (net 7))
 (segment (start 131.331 89.85) (end 130.9425 89.85) (width 0.25) (layer "F.Cu") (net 3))
 (segment (start 128.3021 88.0642) (end 129.1007 87.2656) (width 0.25) (layer "F.Cu") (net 3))
 (segment (start 124.18 86.36) (end 125.8842 88.0642) (width 0.25) (layer "F.Cu") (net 3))
 (segment (start 131.9626 87.5817) (end 131.9626 89.2184) (width 0.25) (layer "F.Cu") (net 3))
 (segment (start 131.9626 89.2184) (end 131.331 89.85) (width 0.25) (layer "F.Cu") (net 3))
 (segment (start 125.8842 88.0642) (end 128.3021 88.0642) (width 0.25) (layer "F.Cu") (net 3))
 (segment (start 127.28 91.44) (end 128.87 89.85) (width 0.25) (layer "F.Cu") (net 3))
 (segment (start 129.1007 87.2656) (end 131.6465 87.2656) (width 0.25) (layer "F.Cu") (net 3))
 (segment (start 128.87 89.85) (end 130.9425 89.85) (width 0.25) (layer "F.Cu") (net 3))
 (segment (start 131.6465 87.2656) (end 131.9626 87.5817) (width 0.25) (layer "F.Cu") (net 3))
 (segment (start 118.5506 95.47) (end 118.5506 95.3885) (width 0.25) (layer "F.Cu") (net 10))
 (segment (start 118.5506 95.3885) (end 115.9599 92.7978) (width 0.25) (layer "F.Cu") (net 10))
 (segment (start 119.2025 95.47) (end 118.5506 95.47) (width 0.25) (layer "F.Cu") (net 10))
 (segment (start 115.9599 92.7978) (end 106.0225 92.7978) (width 0.25) (layer "F.Cu") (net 10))
 (via (at 106.0225 92.7978) (size 0.8) (drill 0.4) (layers "F.Cu" "B.Cu") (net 10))
 (segment (start 106.0225 90.21) (end 106.0225 92.7978) (width 0.25) (layer "B.Cu") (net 10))
 (segment (start 115.8864 96.2142) (end 116.6306 95.47) (width 0.25) (layer "F.Cu") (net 11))
 (segment (start 117.2825 95.47) (end 116.6306 95.47) (width 0.25) (layer "F.Cu") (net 11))
 (segment (start 111.3078 96.2142) (end 115.8864 96.2142) (width 0.25) (layer "F.Cu") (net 11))
 (via (at 111.3078 96.2142) (size 0.8) (drill 0.4) (layers "F.Cu" "B.Cu") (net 11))
 (segment (start 111.3078 91.4453) (end 111.3078 96.2142) (width 0.25) (layer "B.Cu") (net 11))
 (segment (start 106.0225 86.16) (end 111.3078 91.4453) (width 0.25) (layer "B.Cu") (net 11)))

